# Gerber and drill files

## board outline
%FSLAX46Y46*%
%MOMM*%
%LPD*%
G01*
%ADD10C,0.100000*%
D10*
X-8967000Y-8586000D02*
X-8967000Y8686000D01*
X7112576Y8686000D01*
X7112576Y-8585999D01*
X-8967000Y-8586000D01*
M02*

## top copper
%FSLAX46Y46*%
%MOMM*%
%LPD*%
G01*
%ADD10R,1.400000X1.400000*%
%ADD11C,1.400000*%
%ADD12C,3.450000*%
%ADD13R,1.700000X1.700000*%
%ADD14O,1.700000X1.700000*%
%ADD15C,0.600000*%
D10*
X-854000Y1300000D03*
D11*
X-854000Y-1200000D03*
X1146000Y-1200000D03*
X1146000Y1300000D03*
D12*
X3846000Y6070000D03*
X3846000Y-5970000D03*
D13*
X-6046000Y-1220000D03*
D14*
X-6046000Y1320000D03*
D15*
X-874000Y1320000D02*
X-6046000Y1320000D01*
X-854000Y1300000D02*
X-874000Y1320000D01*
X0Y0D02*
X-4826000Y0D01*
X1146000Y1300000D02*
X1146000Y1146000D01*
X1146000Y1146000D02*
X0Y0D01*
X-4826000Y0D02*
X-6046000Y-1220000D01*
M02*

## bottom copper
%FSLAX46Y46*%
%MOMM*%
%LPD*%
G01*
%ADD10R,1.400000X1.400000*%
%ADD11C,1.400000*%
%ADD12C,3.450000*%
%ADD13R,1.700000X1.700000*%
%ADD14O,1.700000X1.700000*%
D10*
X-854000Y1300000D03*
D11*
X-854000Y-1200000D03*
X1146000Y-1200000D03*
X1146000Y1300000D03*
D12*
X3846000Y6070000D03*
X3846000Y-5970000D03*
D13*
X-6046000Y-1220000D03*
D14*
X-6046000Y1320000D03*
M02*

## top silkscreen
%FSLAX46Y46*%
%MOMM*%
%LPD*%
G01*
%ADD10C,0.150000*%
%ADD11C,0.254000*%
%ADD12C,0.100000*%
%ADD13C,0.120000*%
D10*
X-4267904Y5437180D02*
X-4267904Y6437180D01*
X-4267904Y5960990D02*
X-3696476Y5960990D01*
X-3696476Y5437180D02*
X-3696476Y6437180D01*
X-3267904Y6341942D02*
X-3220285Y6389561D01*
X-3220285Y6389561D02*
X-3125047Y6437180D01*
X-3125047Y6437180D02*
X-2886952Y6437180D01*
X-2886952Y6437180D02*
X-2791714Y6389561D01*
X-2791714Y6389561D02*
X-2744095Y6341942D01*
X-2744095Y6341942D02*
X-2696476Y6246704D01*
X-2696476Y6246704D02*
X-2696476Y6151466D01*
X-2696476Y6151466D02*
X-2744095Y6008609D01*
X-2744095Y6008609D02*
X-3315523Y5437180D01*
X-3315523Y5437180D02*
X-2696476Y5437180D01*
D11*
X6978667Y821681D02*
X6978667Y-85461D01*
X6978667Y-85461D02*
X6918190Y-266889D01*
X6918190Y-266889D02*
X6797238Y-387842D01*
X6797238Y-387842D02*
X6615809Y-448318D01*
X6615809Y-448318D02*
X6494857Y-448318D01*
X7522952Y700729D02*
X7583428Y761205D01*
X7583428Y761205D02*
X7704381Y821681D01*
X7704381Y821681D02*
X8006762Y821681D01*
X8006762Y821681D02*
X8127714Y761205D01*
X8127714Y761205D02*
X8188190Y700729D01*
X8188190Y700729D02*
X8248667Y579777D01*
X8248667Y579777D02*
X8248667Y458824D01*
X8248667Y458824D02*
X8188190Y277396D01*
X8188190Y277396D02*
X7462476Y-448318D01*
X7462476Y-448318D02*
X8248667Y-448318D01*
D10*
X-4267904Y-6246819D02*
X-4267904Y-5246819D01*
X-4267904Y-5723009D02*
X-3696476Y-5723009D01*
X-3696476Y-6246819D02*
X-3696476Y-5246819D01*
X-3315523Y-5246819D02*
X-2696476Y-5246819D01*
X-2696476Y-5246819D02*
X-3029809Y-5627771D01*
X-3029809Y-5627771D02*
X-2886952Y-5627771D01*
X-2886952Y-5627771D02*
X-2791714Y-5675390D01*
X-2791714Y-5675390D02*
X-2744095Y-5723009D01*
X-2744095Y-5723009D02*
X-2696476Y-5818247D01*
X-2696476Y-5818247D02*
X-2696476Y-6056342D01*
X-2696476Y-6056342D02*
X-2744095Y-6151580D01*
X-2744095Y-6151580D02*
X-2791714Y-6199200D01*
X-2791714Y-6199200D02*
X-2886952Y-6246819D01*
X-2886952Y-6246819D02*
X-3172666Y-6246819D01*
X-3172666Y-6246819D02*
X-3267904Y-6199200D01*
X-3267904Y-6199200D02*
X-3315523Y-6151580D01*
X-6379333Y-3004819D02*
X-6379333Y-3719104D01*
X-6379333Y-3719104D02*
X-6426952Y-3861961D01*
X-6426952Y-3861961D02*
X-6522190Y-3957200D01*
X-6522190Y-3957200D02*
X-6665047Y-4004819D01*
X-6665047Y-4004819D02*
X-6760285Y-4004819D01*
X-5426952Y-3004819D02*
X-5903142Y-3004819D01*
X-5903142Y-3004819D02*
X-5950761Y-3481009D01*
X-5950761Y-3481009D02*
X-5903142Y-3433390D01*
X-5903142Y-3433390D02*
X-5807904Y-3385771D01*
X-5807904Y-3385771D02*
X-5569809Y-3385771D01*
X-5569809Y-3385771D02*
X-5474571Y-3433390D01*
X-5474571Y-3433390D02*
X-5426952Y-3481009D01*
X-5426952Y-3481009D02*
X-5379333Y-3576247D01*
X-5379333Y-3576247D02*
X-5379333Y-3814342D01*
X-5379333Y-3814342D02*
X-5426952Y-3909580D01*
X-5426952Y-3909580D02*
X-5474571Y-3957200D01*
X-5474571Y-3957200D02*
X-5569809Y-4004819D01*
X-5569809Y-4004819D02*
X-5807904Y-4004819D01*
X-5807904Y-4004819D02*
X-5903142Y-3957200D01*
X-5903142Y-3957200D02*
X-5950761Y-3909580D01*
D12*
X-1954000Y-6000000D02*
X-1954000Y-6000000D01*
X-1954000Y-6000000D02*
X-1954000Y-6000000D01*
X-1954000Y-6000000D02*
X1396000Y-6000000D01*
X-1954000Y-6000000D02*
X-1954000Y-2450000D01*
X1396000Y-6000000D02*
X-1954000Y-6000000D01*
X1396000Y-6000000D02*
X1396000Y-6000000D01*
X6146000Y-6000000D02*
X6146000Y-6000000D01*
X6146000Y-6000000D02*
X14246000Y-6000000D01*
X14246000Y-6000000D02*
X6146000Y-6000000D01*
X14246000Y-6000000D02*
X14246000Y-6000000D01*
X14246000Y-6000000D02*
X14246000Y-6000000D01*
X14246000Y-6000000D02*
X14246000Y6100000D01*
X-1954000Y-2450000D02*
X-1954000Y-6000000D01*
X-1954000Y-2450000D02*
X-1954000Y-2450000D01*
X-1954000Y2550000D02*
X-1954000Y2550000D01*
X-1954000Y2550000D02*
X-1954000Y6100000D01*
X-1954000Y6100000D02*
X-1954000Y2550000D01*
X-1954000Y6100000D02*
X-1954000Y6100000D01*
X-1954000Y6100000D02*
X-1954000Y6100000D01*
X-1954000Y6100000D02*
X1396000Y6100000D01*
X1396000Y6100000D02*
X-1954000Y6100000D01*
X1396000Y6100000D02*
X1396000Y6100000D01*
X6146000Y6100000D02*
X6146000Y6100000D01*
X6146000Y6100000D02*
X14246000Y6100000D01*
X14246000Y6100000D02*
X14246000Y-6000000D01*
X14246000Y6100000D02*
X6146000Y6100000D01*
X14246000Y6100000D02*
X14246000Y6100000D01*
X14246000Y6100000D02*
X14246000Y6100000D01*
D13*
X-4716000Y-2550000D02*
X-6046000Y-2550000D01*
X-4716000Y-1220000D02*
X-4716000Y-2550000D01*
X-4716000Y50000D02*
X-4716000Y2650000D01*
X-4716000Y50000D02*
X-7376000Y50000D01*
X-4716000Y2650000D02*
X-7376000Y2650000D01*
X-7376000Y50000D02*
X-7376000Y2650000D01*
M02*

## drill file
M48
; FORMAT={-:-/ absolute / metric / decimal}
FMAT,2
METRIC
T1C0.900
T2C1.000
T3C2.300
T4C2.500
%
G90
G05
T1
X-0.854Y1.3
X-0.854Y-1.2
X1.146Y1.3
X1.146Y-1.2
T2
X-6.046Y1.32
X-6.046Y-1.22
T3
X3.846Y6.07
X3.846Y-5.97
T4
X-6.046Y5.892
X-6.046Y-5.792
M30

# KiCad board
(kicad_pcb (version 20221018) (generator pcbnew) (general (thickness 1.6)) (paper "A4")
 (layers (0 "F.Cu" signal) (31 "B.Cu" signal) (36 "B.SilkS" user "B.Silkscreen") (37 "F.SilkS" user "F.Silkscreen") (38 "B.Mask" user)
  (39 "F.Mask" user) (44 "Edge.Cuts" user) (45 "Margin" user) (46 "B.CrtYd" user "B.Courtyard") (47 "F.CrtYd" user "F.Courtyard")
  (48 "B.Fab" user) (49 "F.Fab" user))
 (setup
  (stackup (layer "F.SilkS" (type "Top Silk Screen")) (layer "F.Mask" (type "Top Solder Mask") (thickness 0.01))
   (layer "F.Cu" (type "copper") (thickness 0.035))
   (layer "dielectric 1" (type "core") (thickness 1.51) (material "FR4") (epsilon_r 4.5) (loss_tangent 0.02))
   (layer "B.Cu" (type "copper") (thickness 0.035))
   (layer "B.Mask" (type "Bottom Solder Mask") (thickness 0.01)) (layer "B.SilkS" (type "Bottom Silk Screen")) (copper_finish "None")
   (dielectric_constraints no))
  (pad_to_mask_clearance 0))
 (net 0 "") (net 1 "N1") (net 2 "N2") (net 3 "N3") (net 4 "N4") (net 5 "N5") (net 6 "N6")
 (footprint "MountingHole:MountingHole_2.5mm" (layer "F.Cu") (at -6.046 -5.892)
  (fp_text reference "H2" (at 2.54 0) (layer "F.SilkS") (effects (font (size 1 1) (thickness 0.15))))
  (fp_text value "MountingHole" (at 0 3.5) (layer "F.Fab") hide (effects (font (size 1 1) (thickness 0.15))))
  (pad "" np_thru_hole circle (at 0 0) (size 2.5 2.5) (drill 2.5) (layers "*.Cu" "*.Mask")))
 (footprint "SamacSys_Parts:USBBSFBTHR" (layer "F.Cu") (at -0.854 -1.3 90)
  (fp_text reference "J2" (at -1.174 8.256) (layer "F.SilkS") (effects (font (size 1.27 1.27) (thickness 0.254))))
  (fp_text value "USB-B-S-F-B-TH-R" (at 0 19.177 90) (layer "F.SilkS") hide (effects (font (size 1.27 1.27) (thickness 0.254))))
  (fp_line (start -7.3 -1.1) (end -7.3 -1.1) (stroke (width 0.1) (type solid)) (layer "F.SilkS"))
  (fp_line (start -7.3 -1.1) (end -7.3 -1.1) (stroke (width 0.1) (type solid)) (layer "F.SilkS"))
  (fp_line (start -7.3 -1.1) (end -7.3 2.25) (stroke (width 0.1) (type solid)) (layer "F.SilkS"))
  (fp_line (start -7.3 -1.1) (end -3.75 -1.1) (stroke (width 0.1) (type solid)) (layer "F.SilkS"))
  (fp_line (start -7.3 2.25) (end -7.3 -1.1) (stroke (width 0.1) (type solid)) (layer "F.SilkS"))
  (fp_line (start -7.3 2.25) (end -7.3 2.25) (stroke (width 0.1) (type solid)) (layer "F.SilkS"))
  (fp_line (start -7.3 7) (end -7.3 7) (stroke (width 0.1) (type solid)) (layer "F.SilkS"))
  (fp_line (start -7.3 7) (end -7.3 15.1) (stroke (width 0.1) (type solid)) (layer "F.SilkS"))
  (fp_line (start -7.3 15.1) (end -7.3 7) (stroke (width 0.1) (type solid)) (layer "F.SilkS"))
  (fp_line (start -7.3 15.1) (end -7.3 15.1) (stroke (width 0.1) (type solid)) (layer "F.SilkS"))
  (fp_line (start -7.3 15.1) (end -7.3 15.1) (stroke (width 0.1) (type solid)) (layer "F.SilkS"))
  (fp_line (start -7.3 15.1) (end 4.8 15.1) (stroke (width 0.1) (type solid)) (layer "F.SilkS"))
  (fp_line (start -3.75 -1.1) (end -7.3 -1.1) (stroke (width 0.1) (type solid)) (layer "F.SilkS"))
  (fp_line (start -3.75 -1.1) (end -3.75 -1.1) (stroke (width 0.1) (type solid)) (layer "F.SilkS"))
  (fp_line (start 1.25 -1.1) (end 1.25 -1.1) (stroke (width 0.1) (type solid)) (layer "F.SilkS"))
  (fp_line (start 1.25 -1.1) (end 4.8 -1.1) (stroke (width 0.1) (type solid)) (layer "F.SilkS"))
  (fp_line (start 4.8 -1.1) (end 1.25 -1.1) (stroke (width 0.1) (type solid)) (layer "F.SilkS"))
  (fp_line (start 4.8 -1.1) (end 4.8 -1.1) (stroke (width 0.1) (type solid)) (layer "F.SilkS"))
  (fp_line (start 4.8 -1.1) (end 4.8 -1.1) (stroke (width 0.1) (type solid)) (layer "F.SilkS"))
  (fp_line (start 4.8 -1.1) (end 4.8 2.25) (stroke (width 0.1) (type solid)) (layer "F.SilkS"))
  (fp_line (start 4.8 2.25) (end 4.8 -1.1) (stroke (width 0.1) (type solid)) (layer "F.SilkS"))
  (fp_line (start 4.8 2.25) (end 4.8 2.25) (stroke (width 0.1) (type solid)) (layer "F.SilkS"))
  (fp_line (start 4.8 7) (end 4.8 7) (stroke (width 0.1) (type solid)) (layer "F.SilkS"))
  (fp_line (start 4.8 7) (end 4.8 15.1) (stroke (width 0.1) (type solid)) (layer "F.SilkS"))
  (fp_line (start 4.8 15.1) (end -7.3 15.1) (stroke (width 0.1) (type solid)) (layer "F.SilkS"))
  (fp_line (start 4.8 15.1) (end 4.8 7) (stroke (width 0.1) (type solid)) (layer "F.SilkS"))
  (fp_line (start 4.8 15.1) (end 4.8 15.1) (stroke (width 0.1) (type solid)) (layer "F.SilkS"))
  (fp_line (start 4.8 15.1) (end 4.8 15.1) (stroke (width 0.1) (type solid)) (layer "F.SilkS"))
  (pad "1" thru_hole rect (at 0 0 90) (size 1.4 1.4) (drill 0.9) (layers "*.Cu" "*.Mask") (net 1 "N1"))
  (pad "2" thru_hole circle (at -2.5 0 90) (size 1.4 1.4) (drill 0.9) (layers "*.Cu" "*.Mask") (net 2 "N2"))
  (pad "3" thru_hole circle (at -2.5 2 90) (size 1.4 1.4) (drill 0.9) (layers "*.Cu" "*.Mask") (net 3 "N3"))
  (pad "4" thru_hole circle (at 0 2 90) (size 1.4 1.4) (drill 0.9) (layers "*.Cu" "*.Mask") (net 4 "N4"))
  (pad "MH1" thru_hole circle (at 4.77 4.7 90) (size 3.45 3.45) (drill 2.3) (layers "*.Cu" "*.Mask") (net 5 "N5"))
  (pad "MH2" thru_hole circle (at -7.27 4.7 90) (size 3.45 3.45) (drill 2.3) (layers "*.Cu" "*.Mask") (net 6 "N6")))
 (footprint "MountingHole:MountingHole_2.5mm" (layer "F.Cu") (at -6.046 5.792)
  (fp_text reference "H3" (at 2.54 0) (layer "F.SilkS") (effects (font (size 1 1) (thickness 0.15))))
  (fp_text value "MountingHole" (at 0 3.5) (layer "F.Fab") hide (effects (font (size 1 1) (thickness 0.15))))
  (pad "" np_thru_hole circle (at 0 0) (size 2.5 2.5) (drill 2.5) (layers "*.Cu" "*.Mask")))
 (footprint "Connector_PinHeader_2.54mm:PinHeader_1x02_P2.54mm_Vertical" (layer "F.Cu") (at -6.046 1.22 180)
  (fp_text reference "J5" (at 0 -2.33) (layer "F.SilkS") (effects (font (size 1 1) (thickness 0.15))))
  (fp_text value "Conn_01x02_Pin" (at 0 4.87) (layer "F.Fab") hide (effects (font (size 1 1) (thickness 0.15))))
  (fp_line (start -1.33 -1.33) (end 0 -1.33) (stroke (width 0.12) (type solid)) (layer "F.SilkS"))
  (fp_line (start -1.33 0) (end -1.33 -1.33) (stroke (width 0.12) (type solid)) (layer "F.SilkS"))
  (fp_line (start -1.33 1.27) (end -1.33 3.87) (stroke (width 0.12) (type solid)) (layer "F.SilkS"))
  (fp_line (start -1.33 1.27) (end 1.33 1.27) (stroke (width 0.12) (type solid)) (layer "F.SilkS"))
  (fp_line (start -1.33 3.87) (end 1.33 3.87) (stroke (width 0.12) (type solid)) (layer "F.SilkS"))
  (fp_line (start 1.33 1.27) (end 1.33 3.87) (stroke (width 0.12) (type solid)) (layer "F.SilkS"))
  (pad "1" thru_hole rect (at 0 0 180) (size 1.7 1.7) (drill 1) (layers "*.Cu" "*.Mask") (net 4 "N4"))
  (pad "2" thru_hole oval (at 0 2.54 180) (size 1.7 1.7) (drill 1) (layers "*.Cu" "*.Mask") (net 1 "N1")))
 (gr_poly
  (pts (xy -8.967 8.586) (xy -8.967 -8.686) (xy 7.112576 -8.686) (xy 7.112576 8.585999)) (stroke (width 0.1) (type default)) (fill none)
  (layer "Edge.Cuts"))
 (segment (start -0.874 -1.32) (end -6.046 -1.32) (width 0.6) (layer "F.Cu") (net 1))
 (segment (start -0.854 -1.3) (end -0.874 -1.32) (width 0.6) (layer "F.Cu") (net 1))
 (segment (start 0 0) (end -4.826 0) (width 0.6) (layer "F.Cu") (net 4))
 (segment (start 1.146 -1.3) (end 1.146 -1.146) (width 0.6) (layer "F.Cu") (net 4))
 (segment (start 1.146 -1.146) (end 0 0) (width 0.6) (layer "F.Cu") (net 4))
 (segment (start -4.826 0) (end -6.046 1.22) (width 0.6) (layer "F.Cu") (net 4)))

